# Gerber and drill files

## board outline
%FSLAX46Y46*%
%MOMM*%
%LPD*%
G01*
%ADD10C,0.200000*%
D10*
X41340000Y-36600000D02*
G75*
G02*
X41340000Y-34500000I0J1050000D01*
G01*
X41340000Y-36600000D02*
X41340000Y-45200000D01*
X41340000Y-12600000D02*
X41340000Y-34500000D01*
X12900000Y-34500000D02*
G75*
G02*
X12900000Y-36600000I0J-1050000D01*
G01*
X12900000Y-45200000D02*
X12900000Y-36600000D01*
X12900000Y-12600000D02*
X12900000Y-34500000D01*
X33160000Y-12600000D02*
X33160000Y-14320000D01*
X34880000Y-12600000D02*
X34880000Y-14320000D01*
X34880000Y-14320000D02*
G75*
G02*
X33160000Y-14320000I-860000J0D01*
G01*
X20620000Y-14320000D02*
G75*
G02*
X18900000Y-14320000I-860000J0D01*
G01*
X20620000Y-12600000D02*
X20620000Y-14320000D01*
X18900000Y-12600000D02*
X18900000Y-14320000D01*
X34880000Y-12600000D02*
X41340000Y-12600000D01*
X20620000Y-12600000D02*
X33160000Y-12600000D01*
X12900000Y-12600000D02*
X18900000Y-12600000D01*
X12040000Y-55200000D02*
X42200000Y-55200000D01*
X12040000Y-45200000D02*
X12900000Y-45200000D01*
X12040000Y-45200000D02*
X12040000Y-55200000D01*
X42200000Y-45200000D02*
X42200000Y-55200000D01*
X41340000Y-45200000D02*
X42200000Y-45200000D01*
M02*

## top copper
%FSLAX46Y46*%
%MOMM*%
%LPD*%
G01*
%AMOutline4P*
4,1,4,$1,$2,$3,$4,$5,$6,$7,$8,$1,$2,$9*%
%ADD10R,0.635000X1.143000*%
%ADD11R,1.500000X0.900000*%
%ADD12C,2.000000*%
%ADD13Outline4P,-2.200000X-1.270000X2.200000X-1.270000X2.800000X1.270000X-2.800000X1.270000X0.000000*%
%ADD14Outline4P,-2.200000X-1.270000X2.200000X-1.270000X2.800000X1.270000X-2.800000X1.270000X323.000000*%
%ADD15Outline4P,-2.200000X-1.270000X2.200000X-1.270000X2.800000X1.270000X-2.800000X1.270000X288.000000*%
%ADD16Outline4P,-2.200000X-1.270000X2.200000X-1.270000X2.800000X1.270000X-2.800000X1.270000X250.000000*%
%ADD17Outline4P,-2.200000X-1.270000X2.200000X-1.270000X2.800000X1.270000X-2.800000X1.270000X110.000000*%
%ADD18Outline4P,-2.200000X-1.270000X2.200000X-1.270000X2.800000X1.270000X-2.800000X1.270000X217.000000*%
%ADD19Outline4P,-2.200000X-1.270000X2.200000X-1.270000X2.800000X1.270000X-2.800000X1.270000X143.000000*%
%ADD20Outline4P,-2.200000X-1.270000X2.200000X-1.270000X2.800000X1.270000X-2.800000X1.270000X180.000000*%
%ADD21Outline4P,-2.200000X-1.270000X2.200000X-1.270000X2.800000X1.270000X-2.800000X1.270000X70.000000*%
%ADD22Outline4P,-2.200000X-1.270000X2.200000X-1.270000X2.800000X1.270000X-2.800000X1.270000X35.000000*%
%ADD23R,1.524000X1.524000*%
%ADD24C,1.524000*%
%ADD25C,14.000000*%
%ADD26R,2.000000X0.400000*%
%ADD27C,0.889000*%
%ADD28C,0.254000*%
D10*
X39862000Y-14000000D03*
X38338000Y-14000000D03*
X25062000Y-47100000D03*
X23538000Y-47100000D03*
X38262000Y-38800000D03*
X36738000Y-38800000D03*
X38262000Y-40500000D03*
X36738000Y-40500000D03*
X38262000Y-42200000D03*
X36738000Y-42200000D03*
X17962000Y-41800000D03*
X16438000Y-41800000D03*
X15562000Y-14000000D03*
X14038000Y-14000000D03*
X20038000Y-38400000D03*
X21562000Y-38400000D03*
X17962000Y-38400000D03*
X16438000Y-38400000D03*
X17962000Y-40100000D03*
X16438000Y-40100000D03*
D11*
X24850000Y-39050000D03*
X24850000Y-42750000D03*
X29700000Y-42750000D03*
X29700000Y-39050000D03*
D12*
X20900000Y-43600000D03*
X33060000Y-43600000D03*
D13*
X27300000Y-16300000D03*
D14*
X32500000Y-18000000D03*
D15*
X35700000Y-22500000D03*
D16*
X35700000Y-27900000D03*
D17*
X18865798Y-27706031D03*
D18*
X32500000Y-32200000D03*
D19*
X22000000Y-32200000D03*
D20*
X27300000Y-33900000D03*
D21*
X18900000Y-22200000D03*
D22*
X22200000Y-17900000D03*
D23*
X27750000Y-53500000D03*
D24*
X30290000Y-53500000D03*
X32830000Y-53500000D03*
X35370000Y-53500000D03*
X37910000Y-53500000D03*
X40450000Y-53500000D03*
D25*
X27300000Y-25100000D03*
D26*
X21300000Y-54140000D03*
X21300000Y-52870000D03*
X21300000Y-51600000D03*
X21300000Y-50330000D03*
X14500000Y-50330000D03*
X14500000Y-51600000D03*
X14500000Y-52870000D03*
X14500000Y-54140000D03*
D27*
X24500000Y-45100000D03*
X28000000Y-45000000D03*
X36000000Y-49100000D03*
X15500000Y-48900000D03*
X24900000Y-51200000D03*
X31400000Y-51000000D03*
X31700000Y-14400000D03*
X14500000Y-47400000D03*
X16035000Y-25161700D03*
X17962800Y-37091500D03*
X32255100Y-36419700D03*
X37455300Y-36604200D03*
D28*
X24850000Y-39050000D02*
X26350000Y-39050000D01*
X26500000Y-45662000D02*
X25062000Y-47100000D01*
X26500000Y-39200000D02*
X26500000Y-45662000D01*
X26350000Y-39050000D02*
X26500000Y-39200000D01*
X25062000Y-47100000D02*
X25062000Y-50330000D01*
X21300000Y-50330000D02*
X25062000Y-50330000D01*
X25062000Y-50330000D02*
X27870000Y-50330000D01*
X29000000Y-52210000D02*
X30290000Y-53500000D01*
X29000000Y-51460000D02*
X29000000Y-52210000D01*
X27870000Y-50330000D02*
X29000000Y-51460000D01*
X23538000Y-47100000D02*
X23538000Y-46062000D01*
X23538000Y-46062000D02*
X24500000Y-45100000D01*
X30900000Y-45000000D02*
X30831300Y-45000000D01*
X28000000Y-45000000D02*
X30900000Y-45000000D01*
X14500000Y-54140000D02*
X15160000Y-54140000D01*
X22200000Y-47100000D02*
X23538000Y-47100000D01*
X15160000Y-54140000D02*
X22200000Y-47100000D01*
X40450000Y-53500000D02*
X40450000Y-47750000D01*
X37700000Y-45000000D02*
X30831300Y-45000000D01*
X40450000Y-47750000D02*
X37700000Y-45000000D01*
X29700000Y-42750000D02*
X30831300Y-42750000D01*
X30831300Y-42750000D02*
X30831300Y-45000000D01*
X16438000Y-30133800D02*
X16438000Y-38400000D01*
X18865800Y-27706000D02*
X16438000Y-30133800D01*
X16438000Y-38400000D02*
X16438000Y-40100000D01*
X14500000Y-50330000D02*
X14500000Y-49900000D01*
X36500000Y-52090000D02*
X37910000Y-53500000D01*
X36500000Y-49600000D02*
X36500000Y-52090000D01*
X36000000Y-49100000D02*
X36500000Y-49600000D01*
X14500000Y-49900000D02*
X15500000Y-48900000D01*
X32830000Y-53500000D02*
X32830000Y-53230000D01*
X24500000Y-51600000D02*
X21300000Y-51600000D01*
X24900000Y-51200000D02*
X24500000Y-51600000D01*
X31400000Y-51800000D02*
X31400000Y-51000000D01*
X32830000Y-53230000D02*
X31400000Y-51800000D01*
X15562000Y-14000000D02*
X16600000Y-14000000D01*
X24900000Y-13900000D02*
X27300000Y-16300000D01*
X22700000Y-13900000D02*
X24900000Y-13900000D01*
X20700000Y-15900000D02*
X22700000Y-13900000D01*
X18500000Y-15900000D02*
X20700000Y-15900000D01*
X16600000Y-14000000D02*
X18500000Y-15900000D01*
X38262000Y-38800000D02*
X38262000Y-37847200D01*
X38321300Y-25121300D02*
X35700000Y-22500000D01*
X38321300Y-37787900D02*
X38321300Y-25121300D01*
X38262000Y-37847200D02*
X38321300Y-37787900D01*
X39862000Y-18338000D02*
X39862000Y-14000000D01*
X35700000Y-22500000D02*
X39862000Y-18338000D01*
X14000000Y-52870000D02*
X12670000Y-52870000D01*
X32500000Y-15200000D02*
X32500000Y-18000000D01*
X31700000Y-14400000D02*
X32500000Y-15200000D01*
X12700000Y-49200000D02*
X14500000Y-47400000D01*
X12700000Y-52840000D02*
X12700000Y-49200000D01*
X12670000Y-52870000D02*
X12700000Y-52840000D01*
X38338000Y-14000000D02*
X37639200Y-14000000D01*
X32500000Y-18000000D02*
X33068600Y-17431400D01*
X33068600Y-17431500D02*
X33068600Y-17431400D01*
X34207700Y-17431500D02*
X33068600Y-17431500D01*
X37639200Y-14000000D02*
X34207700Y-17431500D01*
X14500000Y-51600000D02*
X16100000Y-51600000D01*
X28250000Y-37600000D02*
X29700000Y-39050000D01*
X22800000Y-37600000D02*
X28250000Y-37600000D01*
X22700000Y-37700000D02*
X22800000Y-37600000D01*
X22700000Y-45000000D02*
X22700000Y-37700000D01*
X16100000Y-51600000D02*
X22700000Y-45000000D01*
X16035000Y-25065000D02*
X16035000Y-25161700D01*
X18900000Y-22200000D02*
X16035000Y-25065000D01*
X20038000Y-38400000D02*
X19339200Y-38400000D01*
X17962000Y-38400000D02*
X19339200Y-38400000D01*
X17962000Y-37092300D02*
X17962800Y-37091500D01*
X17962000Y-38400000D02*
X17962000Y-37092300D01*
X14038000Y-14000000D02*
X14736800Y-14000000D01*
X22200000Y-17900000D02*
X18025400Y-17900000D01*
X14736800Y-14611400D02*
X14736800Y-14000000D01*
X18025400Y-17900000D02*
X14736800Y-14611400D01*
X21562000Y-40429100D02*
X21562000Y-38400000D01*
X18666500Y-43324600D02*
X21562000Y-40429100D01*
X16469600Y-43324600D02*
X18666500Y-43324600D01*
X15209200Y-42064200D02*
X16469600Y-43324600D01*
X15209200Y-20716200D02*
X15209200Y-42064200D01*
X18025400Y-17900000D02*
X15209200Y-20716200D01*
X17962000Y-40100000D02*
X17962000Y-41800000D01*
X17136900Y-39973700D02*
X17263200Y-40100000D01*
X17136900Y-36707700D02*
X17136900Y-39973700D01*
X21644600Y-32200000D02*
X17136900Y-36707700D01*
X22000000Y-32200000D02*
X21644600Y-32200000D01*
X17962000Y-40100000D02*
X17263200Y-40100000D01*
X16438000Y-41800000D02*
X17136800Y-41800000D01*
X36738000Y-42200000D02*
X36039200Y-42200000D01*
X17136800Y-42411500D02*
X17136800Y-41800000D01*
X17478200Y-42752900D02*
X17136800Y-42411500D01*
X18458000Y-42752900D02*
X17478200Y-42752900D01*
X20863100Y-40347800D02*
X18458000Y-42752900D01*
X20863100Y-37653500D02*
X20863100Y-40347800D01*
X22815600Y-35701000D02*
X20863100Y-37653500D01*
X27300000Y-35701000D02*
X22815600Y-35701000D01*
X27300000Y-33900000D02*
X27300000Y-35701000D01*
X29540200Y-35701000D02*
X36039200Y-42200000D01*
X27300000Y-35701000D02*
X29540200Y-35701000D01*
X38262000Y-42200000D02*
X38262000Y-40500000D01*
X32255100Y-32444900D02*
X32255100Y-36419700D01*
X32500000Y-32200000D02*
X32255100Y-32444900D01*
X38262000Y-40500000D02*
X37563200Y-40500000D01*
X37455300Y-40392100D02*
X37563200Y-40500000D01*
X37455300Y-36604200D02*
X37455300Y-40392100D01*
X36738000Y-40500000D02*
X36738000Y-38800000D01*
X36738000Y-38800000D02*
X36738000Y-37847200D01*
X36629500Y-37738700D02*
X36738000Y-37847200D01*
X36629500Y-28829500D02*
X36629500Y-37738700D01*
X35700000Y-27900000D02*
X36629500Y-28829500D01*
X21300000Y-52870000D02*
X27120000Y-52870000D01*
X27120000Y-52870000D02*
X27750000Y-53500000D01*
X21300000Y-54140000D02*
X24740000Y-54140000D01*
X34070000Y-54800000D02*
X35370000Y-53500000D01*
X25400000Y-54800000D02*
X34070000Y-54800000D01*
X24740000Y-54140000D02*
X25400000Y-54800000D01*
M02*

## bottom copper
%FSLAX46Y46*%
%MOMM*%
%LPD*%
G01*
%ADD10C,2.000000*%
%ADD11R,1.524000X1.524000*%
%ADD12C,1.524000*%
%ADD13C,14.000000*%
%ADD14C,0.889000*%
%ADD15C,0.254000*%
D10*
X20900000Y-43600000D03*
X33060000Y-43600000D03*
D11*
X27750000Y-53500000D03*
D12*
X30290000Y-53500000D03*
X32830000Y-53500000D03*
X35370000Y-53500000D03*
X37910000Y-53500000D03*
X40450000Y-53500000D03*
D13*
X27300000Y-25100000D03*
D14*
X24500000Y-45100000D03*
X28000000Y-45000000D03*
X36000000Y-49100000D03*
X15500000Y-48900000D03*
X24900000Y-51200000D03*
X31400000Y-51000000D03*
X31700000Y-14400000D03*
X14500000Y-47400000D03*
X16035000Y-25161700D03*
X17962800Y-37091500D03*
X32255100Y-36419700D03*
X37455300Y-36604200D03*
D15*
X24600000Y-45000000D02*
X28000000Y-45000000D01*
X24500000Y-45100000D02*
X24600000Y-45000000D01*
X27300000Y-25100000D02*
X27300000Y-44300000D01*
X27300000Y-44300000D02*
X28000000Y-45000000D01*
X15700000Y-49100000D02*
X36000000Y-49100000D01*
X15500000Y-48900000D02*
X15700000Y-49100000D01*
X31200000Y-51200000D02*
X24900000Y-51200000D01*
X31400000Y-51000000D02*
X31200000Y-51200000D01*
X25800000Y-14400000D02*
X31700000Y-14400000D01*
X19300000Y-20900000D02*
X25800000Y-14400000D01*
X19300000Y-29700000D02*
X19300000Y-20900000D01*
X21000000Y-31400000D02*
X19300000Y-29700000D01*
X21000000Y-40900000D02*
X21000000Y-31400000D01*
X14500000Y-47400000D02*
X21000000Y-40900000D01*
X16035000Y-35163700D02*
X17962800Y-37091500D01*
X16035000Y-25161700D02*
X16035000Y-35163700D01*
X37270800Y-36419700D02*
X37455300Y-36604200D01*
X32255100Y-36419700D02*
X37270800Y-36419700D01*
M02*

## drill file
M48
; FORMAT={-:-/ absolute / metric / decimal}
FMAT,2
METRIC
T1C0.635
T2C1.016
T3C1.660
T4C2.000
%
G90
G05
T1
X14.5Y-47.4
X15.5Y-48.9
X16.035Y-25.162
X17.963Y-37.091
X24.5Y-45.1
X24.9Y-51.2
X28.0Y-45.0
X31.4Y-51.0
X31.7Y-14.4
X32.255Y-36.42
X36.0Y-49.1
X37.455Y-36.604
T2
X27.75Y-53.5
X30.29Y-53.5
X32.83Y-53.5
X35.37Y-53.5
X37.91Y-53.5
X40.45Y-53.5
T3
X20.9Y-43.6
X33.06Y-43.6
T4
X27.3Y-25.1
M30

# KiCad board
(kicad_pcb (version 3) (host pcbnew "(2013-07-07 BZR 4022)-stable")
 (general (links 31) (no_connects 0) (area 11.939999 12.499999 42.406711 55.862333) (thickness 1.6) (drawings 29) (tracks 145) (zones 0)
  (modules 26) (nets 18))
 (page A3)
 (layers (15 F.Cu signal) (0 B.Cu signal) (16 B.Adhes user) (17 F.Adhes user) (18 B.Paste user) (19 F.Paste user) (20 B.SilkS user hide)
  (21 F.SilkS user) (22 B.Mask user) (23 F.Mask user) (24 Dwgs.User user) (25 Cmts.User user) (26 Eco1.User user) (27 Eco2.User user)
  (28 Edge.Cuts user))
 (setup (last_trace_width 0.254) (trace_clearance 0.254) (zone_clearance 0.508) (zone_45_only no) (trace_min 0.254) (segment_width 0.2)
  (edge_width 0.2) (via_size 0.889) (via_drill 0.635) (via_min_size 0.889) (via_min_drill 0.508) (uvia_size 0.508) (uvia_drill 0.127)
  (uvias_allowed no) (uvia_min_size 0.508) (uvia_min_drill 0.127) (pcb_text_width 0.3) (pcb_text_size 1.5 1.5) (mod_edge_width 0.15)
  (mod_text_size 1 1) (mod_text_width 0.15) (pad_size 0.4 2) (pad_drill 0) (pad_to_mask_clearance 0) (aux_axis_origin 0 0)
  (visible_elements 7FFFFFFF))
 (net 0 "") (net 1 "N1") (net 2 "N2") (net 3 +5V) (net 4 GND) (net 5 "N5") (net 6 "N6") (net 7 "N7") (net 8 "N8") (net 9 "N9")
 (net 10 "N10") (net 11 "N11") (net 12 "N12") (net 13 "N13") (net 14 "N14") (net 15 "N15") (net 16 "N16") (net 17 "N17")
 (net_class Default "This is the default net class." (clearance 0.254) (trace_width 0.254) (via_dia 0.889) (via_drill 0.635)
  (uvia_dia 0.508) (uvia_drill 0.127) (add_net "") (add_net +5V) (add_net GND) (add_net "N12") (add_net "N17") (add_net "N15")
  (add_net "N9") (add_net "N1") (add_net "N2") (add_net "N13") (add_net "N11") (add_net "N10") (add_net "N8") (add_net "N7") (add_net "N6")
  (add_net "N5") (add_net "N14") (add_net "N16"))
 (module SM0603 (layer F.Cu) (at 39.1 14 180)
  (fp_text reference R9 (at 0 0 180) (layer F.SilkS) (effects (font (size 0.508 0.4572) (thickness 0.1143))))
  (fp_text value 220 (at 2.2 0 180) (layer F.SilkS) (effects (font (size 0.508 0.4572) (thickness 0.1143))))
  (pad 1 smd rect (at -0.762 0 180) (size 0.635 1.143) (layers F.Cu F.Paste F.Mask) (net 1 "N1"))
  (pad 2 smd rect (at 0.762 0 180) (size 0.635 1.143) (layers F.Cu F.Paste F.Mask) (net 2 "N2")))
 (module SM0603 (layer F.Cu) (at 24.3 47.1 180)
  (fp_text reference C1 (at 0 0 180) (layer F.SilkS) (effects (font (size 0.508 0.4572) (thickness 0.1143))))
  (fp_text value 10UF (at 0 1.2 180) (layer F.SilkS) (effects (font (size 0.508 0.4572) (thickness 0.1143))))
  (pad 1 smd rect (at -0.762 0 180) (size 0.635 1.143) (layers F.Cu F.Paste F.Mask) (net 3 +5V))
  (pad 2 smd rect (at 0.762 0 180) (size 0.635 1.143) (layers F.Cu F.Paste F.Mask) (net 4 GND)))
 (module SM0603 (layer F.Cu) (at 37.5 38.8 180)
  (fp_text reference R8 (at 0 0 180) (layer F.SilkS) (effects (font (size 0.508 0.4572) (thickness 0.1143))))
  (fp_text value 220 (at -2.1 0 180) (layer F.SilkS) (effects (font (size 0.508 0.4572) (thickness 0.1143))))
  (pad 1 smd rect (at -0.762 0 180) (size 0.635 1.143) (layers F.Cu F.Paste F.Mask) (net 1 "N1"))
  (pad 2 smd rect (at 0.762 0 180) (size 0.635 1.143) (layers F.Cu F.Paste F.Mask) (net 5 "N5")))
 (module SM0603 (layer F.Cu) (at 37.5 40.5 180)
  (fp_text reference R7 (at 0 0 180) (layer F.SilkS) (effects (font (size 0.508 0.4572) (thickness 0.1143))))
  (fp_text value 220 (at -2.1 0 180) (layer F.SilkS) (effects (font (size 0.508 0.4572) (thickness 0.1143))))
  (pad 1 smd rect (at -0.762 0 180) (size 0.635 1.143) (layers F.Cu F.Paste F.Mask) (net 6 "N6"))
  (pad 2 smd rect (at 0.762 0 180) (size 0.635 1.143) (layers F.Cu F.Paste F.Mask) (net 5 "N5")))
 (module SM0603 (layer F.Cu) (at 37.5 42.2 180)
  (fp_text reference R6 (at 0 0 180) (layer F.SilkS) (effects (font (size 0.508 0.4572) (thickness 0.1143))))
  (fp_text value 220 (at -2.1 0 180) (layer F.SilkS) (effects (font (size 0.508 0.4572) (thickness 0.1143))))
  (pad 1 smd rect (at -0.762 0 180) (size 0.635 1.143) (layers F.Cu F.Paste F.Mask) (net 6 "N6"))
  (pad 2 smd rect (at 0.762 0 180) (size 0.635 1.143) (layers F.Cu F.Paste F.Mask) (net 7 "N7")))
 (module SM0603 (layer F.Cu) (at 17.2 41.8 180)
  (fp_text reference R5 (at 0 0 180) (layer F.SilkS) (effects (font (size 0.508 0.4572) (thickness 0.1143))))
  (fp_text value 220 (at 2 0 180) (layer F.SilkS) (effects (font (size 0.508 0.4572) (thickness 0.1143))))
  (pad 1 smd rect (at -0.762 0 180) (size 0.635 1.143) (layers F.Cu F.Paste F.Mask) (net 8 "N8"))
  (pad 2 smd rect (at 0.762 0 180) (size 0.635 1.143) (layers F.Cu F.Paste F.Mask) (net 7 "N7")))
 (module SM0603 (layer F.Cu) (at 14.8 14 180)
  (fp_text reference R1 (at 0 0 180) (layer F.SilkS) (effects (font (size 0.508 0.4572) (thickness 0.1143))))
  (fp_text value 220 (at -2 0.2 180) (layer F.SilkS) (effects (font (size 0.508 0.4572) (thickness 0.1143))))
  (pad 1 smd rect (at -0.762 0 180) (size 0.635 1.143) (layers F.Cu F.Paste F.Mask) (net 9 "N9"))
  (pad 2 smd rect (at 0.762 0 180) (size 0.635 1.143) (layers F.Cu F.Paste F.Mask) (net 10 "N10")))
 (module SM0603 (layer F.Cu) (at 20.8 38.4)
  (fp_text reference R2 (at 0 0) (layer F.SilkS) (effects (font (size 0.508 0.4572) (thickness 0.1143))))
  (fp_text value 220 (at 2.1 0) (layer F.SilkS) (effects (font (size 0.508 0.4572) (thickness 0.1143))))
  (pad 1 smd rect (at -0.762 0) (size 0.635 1.143) (layers F.Cu F.Paste F.Mask) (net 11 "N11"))
  (pad 2 smd rect (at 0.762 0) (size 0.635 1.143) (layers F.Cu F.Paste F.Mask) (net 10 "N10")))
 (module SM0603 (layer F.Cu) (at 17.2 38.4 180)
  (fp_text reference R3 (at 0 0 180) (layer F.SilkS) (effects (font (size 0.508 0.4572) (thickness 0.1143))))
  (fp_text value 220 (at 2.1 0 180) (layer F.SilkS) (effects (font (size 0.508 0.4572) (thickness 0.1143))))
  (pad 1 smd rect (at -0.762 0 180) (size 0.635 1.143) (layers F.Cu F.Paste F.Mask) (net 11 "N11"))
  (pad 2 smd rect (at 0.762 0 180) (size 0.635 1.143) (layers F.Cu F.Paste F.Mask) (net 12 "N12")))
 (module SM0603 (layer F.Cu) (at 17.2 40.1 180)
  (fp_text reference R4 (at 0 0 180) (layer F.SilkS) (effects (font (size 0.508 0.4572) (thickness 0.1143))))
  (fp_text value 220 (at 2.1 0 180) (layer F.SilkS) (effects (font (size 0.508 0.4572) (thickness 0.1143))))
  (pad 1 smd rect (at -0.762 0 180) (size 0.635 1.143) (layers F.Cu F.Paste F.Mask) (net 8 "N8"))
  (pad 2 smd rect (at 0.762 0 180) (size 0.635 1.143) (layers F.Cu F.Paste F.Mask) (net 12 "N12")))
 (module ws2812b (layer F.Cu) (at 27.3 40.9)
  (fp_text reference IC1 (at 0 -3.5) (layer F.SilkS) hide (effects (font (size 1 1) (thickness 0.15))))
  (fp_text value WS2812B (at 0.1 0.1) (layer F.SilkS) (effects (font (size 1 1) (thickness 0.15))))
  (pad 1 smd rect (at -2.45 -1.85) (size 1.5 0.9) (layers F.Cu F.Paste F.Mask) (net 3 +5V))
  (pad 2 smd rect (at -2.45 1.85) (size 1.5 0.9) (layers F.Cu F.Paste F.Mask))
  (pad 3 smd rect (at 2.4 1.85) (size 1.5 0.9) (layers F.Cu F.Paste F.Mask) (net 4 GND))
  (pad 4 smd rect (at 2.4 -1.85) (size 1.5 0.9) (layers F.Cu F.Paste F.Mask) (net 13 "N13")))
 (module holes (layer F.Cu) (at 20.9 43.6)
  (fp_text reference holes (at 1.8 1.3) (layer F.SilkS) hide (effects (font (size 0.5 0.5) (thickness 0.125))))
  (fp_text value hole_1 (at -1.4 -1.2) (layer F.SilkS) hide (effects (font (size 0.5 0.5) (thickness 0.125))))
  (pad 2 thru_hole circle (at 0 0) (size 2 2) (drill 1.66) (layers *.Cu *.Mask F.SilkS)))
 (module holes (layer F.Cu) (at 33.1 43.6)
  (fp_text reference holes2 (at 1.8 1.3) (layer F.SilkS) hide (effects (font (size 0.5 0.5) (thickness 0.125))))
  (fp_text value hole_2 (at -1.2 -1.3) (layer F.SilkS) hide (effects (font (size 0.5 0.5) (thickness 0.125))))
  (pad 2 thru_hole circle (at -0.04 0) (size 2 2) (drill 1.66) (layers *.Cu *.Mask F.SilkS)))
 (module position (layer F.Cu) (at 27.4 16.3)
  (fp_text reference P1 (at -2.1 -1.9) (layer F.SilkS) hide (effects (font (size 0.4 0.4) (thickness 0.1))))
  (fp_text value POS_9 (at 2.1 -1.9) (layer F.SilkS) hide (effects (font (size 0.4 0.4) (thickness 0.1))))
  (pad 1 smd trapezoid (at -0.1 0) (size 5 2.54) (rect_delta 0 -0.6) (layers F.Cu F.Paste F.Mask) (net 9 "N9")))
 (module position (layer F.Cu) (at 32.5 18 323)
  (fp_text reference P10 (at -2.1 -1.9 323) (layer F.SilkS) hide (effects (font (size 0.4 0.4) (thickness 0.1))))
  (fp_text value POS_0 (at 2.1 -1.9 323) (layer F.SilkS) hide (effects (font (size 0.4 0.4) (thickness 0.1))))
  (pad 1 smd trapezoid (at 0 0 323) (size 5 2.54) (rect_delta 0 -0.6) (layers F.Cu F.Paste F.Mask) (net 2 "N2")))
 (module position (layer F.Cu) (at 35.7 22.5 288)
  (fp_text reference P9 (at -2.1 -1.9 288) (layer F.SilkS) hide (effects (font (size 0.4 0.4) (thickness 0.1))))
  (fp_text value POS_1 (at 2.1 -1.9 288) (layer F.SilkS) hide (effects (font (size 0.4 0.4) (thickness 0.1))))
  (pad 1 smd trapezoid (at 0 0 288) (size 5 2.54) (rect_delta 0 -0.6) (layers F.Cu F.Paste F.Mask) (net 1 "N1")))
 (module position (layer F.Cu) (at 35.7 27.9 250)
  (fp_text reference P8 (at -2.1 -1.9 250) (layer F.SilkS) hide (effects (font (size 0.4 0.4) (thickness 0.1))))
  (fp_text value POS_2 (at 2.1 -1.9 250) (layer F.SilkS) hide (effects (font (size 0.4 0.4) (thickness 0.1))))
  (pad 1 smd trapezoid (at 0 0 250) (size 5 2.54) (rect_delta 0 -0.6) (layers F.Cu F.Paste F.Mask) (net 5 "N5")))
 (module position (layer F.Cu) (at 18.9 27.8 110)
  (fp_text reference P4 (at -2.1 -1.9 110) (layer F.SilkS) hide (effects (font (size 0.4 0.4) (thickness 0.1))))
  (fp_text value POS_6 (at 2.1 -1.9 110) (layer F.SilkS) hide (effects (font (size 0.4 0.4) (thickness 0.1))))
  (pad 1 smd trapezoid (at 0.1 0 110) (size 5 2.54) (rect_delta 0 -0.6) (layers F.Cu F.Paste F.Mask) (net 12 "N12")))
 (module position (layer F.Cu) (at 32.5 32.2 217)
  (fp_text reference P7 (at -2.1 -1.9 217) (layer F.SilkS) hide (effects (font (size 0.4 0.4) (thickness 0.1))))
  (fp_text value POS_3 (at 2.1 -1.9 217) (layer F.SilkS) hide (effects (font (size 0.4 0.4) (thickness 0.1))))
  (pad 1 smd trapezoid (at 0 0 217) (size 5 2.54) (rect_delta 0 -0.6) (layers F.Cu F.Paste F.Mask) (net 6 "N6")))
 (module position (layer F.Cu) (at 22 32.2 143)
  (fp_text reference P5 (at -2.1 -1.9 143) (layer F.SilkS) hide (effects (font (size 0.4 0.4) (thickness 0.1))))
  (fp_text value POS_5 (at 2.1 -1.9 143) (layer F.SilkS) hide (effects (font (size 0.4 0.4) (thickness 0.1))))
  (pad 1 smd trapezoid (at 0 0 143) (size 5 2.54) (rect_delta 0 -0.6) (layers F.Cu F.Paste F.Mask) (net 8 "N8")))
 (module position (layer F.Cu) (at 27.3 33.9 180)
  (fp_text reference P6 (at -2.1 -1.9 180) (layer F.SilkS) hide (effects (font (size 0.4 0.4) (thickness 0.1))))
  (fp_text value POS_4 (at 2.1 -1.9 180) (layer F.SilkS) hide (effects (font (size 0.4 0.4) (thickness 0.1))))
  (pad 1 smd trapezoid (at 0 0 180) (size 5 2.54) (rect_delta 0 -0.6) (layers F.Cu F.Paste F.Mask) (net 7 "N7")))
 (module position (layer F.Cu) (at 18.9 22.2 70)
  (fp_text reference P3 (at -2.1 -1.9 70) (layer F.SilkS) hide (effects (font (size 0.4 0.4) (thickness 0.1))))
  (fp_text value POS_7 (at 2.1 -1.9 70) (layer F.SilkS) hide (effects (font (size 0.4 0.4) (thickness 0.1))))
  (pad 1 smd trapezoid (at 0 0 70) (size 5 2.54) (rect_delta 0 -0.6) (layers F.Cu F.Paste F.Mask) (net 11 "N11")))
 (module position (layer F.Cu) (at 22.2 17.9 35)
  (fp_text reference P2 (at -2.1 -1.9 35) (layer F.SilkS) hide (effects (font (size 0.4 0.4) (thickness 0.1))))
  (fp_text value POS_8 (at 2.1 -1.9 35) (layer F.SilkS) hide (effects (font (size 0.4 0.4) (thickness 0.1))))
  (pad 1 smd trapezoid (at 0 0 35) (size 5 2.54) (rect_delta 0 -0.6) (layers F.Cu F.Paste F.Mask) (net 10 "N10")))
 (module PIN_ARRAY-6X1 (layer F.Cu) (at 34.1 53.5)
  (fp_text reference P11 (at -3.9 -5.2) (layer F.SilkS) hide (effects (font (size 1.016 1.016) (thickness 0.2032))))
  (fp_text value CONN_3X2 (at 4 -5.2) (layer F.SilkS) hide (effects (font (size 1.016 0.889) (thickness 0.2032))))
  (pad 1 thru_hole rect (at -6.35 0) (size 1.524 1.524) (drill 1.016) (layers *.Cu *.Mask F.SilkS) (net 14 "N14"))
  (pad 2 thru_hole circle (at -3.81 0) (size 1.524 1.524) (drill 1.016) (layers *.Cu *.Mask F.SilkS) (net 3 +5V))
  (pad 3 thru_hole circle (at -1.27 0) (size 1.524 1.524) (drill 1.016) (layers *.Cu *.Mask F.SilkS) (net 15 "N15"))
  (pad 4 thru_hole circle (at 1.27 0) (size 1.524 1.524) (drill 1.016) (layers *.Cu *.Mask F.SilkS) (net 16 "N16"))
  (pad 5 thru_hole circle (at 3.81 0) (size 1.524 1.524) (drill 1.016) (layers *.Cu *.Mask F.SilkS) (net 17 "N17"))
  (pad 6 thru_hole circle (at 6.35 0) (size 1.524 1.524) (drill 1.016) (layers *.Cu *.Mask F.SilkS) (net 4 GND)))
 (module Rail (layer F.Cu) (at 27.3 25.1 90)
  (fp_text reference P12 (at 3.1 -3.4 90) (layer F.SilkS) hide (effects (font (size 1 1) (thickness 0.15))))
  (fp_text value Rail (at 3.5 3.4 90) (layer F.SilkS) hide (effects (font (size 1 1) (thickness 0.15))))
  (pad 1 thru_hole circle (at 0 0 90) (size 14 14) (drill 2) (layers *.Cu *.Mask F.SilkS) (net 4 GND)))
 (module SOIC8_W (layer F.Cu) (at 18 52.2 270)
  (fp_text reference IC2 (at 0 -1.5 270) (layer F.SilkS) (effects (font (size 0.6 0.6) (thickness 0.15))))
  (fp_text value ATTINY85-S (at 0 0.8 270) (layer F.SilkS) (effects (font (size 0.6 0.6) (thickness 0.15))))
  (pad 5 smd rect (at 1.94 -3.3 270) (size 0.4 2) (layers F.Cu F.Paste F.Mask) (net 16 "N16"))
  (pad 6 smd rect (at 0.67 -3.3 270) (size 0.4 2) (layers F.Cu F.Paste F.Mask) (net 14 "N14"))
  (pad 7 smd rect (at -0.6 -3.3 270) (size 0.4 2) (layers F.Cu F.Paste F.Mask) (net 15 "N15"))
  (pad 8 smd rect (at -1.87 -3.3 270) (size 0.4 2) (layers F.Cu F.Paste F.Mask) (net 3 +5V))
  (pad 1 smd rect (at -1.87 3.5 270) (size 0.4 2) (layers F.Cu F.Paste F.Mask) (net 17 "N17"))
  (pad 2 smd rect (at -0.6 3.5 270) (size 0.4 2) (layers F.Cu F.Paste F.Mask) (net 13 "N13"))
  (pad 3 smd rect (at 0.67 3.5 270) (size 0.4 2) (layers F.Cu F.Paste F.Mask) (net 2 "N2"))
  (pad 4 smd rect (at 1.94 3.5 270) (size 0.4 2) (layers F.Cu F.Paste F.Mask) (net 4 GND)))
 (gr_arc (start 41.34 35.55) (end 41.34 34.5) (angle -180) (layer Edge.Cuts) (width 0.2))
 (gr_line (start 41.34 36.6) (end 41.34 45.2) (angle 90) (layer Edge.Cuts) (width 0.2))
 (gr_line (start 41.34 12.6) (end 41.34 34.5) (angle 90) (layer Edge.Cuts) (width 0.2))
 (gr_arc (start 12.9 35.55) (end 12.9 34.5) (angle 180) (layer Edge.Cuts) (width 0.2))
 (gr_line (start 12.9 45.2) (end 12.9 36.6) (angle 90) (layer Edge.Cuts) (width 0.2))
 (gr_line (start 12.9 12.6) (end 12.9 34.5) (angle 90) (layer Edge.Cuts) (width 0.2))
 (gr_line (start 33.16 12.6) (end 33.16 14.32) (angle 90) (layer Edge.Cuts) (width 0.2))
 (gr_line (start 34.88 12.6) (end 34.88 14.32) (angle 90) (layer Edge.Cuts) (width 0.2))
 (gr_arc (start 34.02 14.32) (end 33.16 14.32) (angle -180) (layer Edge.Cuts) (width 0.2))
 (gr_arc (start 19.76 14.32) (end 18.9 14.32) (angle -180) (layer Edge.Cuts) (width 0.2))
 (gr_line (start 20.62 12.6) (end 20.62 14.32) (angle 90) (layer Edge.Cuts) (width 0.2))
 (gr_line (start 18.9 12.6) (end 18.9 14.32) (angle 90) (layer Edge.Cuts) (width 0.2))
 (gr_line (start 34.88 12.6) (end 41.34 12.6) (angle 90) (layer Edge.Cuts) (width 0.2))
 (gr_line (start 20.62 12.6) (end 33.16 12.6) (angle 90) (layer Edge.Cuts) (width 0.2))
 (gr_line (start 12.9 12.6) (end 18.9 12.6) (angle 90) (layer Edge.Cuts) (width 0.2))
 (gr_line (start 12.04 55.2) (end 42.2 55.2) (angle 90) (layer Edge.Cuts) (width 0.2))
 (gr_line (start 12.04 45.2) (end 12.9 45.2) (angle 90) (layer Edge.Cuts) (width 0.2))
 (gr_line (start 12.04 45.2) (end 12.04 55.2) (angle 90) (layer Edge.Cuts) (width 0.2))
 (gr_line (start 42.2 45.2) (end 42.2 55.2) (angle 90) (layer Edge.Cuts) (width 0.2))
 (gr_line (start 41.34 45.2) (end 42.2 45.2) (angle 90) (layer Edge.Cuts) (width 0.2))
 (segment (start 24.85 39.05) (end 26.35 39.05) (width 0.254) (layer F.Cu) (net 3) (status 400000))
 (segment (start 26.5 45.662) (end 25.062 47.1) (width 0.254) (layer F.Cu) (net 3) (status 800000))
 (segment (start 26.5 39.2) (end 26.5 45.662) (width 0.254) (layer F.Cu) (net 3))
 (segment (start 26.35 39.05) (end 26.5 39.2) (width 0.254) (layer F.Cu) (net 3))
 (segment (start 25.062 47.1) (end 25.062 50.33) (width 0.254) (layer F.Cu) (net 3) (status 400000))
 (segment (start 21.3 50.33) (end 25.062 50.33) (width 0.254) (layer F.Cu) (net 3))
 (segment (start 25.062 50.33) (end 27.87 50.33) (width 0.254) (layer F.Cu) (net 3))
 (segment (start 29 52.21) (end 30.29 53.5) (width 0.254) (layer F.Cu) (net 3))
 (segment (start 29 51.46) (end 29 52.21) (width 0.254) (layer F.Cu) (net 3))
 (segment (start 27.87 50.33) (end 29 51.46) (width 0.254) (layer F.Cu) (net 3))
 (segment (start 23.538 47.1) (end 23.538 46.062) (width 0.254) (layer F.Cu) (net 4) (status 400000))
 (segment (start 24.6 45) (end 28 45) (width 0.254) (layer B.Cu) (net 4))
 (segment (start 24.5 45.1) (end 24.6 45) (width 0.254) (layer B.Cu) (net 4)) (via (at 24.5 45.1) (size 0.889) (layers F.Cu B.Cu) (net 4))
 (segment (start 23.538 46.062) (end 24.5 45.1) (width 0.254) (layer F.Cu) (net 4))
 (segment (start 27.3 25.1) (end 27.3 44.3) (width 0.254) (layer B.Cu) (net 4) (status 400000))
 (segment (start 27.3 44.3) (end 28 45) (width 0.254) (layer B.Cu) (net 4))
 (segment (start 30.9 45) (end 30.8313 45) (width 0.254) (layer F.Cu) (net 4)) (via (at 28 45) (size 0.889) (layers F.Cu B.Cu) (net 4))
 (segment (start 28 45) (end 30.9 45) (width 0.254) (layer F.Cu) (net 4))
 (segment (start 14.5 54.14) (end 15.16 54.14) (width 0.254) (layer F.Cu) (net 4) (status C00000))
 (segment (start 22.2 47.1) (end 23.538 47.1) (width 0.254) (layer F.Cu) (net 4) (status 800000))
 (segment (start 15.16 54.14) (end 22.2 47.1) (width 0.254) (layer F.Cu) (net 4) (status 400000))
 (segment (start 40.45 53.5) (end 40.45 47.75) (width 0.254) (layer F.Cu) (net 4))
 (segment (start 37.7 45) (end 30.8313 45) (width 0.254) (layer F.Cu) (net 4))
 (segment (start 40.45 47.75) (end 37.7 45) (width 0.254) (layer F.Cu) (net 4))
 (segment (start 29.7 42.75) (end 30.8313 42.75) (width 0.254) (layer F.Cu) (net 4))
 (segment (start 30.8313 42.75) (end 30.8313 45) (width 0.254) (layer F.Cu) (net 4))
 (segment (start 16.438 30.1338) (end 16.438 38.4) (width 0.254) (layer F.Cu) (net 12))
 (segment (start 18.8658 27.706) (end 16.438 30.1338) (width 0.254) (layer F.Cu) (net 12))
 (segment (start 16.438 38.4) (end 16.438 40.1) (width 0.254) (layer F.Cu) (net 12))
 (segment (start 14.5 50.33) (end 14.5 49.9) (width 0.254) (layer F.Cu) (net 17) (status 400000))
 (segment (start 36.5 52.09) (end 37.91 53.5) (width 0.254) (layer F.Cu) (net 17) (status 800000))
 (segment (start 36.5 49.6) (end 36.5 52.09) (width 0.254) (layer F.Cu) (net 17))
 (segment (start 36 49.1) (end 36.5 49.6) (width 0.254) (layer F.Cu) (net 17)) (via (at 36 49.1) (size 0.889) (layers F.Cu B.Cu) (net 17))
 (segment (start 15.7 49.1) (end 36 49.1) (width 0.254) (layer B.Cu) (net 17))
 (segment (start 15.5 48.9) (end 15.7 49.1) (width 0.254) (layer B.Cu) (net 17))
 (via (at 15.5 48.9) (size 0.889) (layers F.Cu B.Cu) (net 17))
 (segment (start 14.5 49.9) (end 15.5 48.9) (width 0.254) (layer F.Cu) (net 17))
 (segment (start 32.83 53.5) (end 32.83 53.23) (width 0.254) (layer F.Cu) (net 15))
 (segment (start 24.5 51.6) (end 21.3 51.6) (width 0.254) (layer F.Cu) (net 15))
 (segment (start 24.9 51.2) (end 24.5 51.6) (width 0.254) (layer F.Cu) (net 15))
 (via (at 24.9 51.2) (size 0.889) (layers F.Cu B.Cu) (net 15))
 (segment (start 31.2 51.2) (end 24.9 51.2) (width 0.254) (layer B.Cu) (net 15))
 (segment (start 31.4 51) (end 31.2 51.2) (width 0.254) (layer B.Cu) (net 15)) (via (at 31.4 51) (size 0.889) (layers F.Cu B.Cu) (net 15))
 (segment (start 31.4 51.8) (end 31.4 51) (width 0.254) (layer F.Cu) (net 15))
 (segment (start 32.83 53.23) (end 31.4 51.8) (width 0.254) (layer F.Cu) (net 15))
 (segment (start 15.562 14) (end 16.6 14) (width 0.254) (layer F.Cu) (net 9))
 (segment (start 24.9 13.9) (end 27.3 16.3) (width 0.254) (layer F.Cu) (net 9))
 (segment (start 22.7 13.9) (end 24.9 13.9) (width 0.254) (layer F.Cu) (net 9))
 (segment (start 20.7 15.9) (end 22.7 13.9) (width 0.254) (layer F.Cu) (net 9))
 (segment (start 18.5 15.9) (end 20.7 15.9) (width 0.254) (layer F.Cu) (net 9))
 (segment (start 16.6 14) (end 18.5 15.9) (width 0.254) (layer F.Cu) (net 9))
 (segment (start 38.262 38.8) (end 38.262 37.8472) (width 0.254) (layer F.Cu) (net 1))
 (segment (start 38.3213 25.1213) (end 35.7 22.5) (width 0.254) (layer F.Cu) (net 1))
 (segment (start 38.3213 37.7879) (end 38.3213 25.1213) (width 0.254) (layer F.Cu) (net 1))
 (segment (start 38.262 37.8472) (end 38.3213 37.7879) (width 0.254) (layer F.Cu) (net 1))
 (segment (start 39.862 18.338) (end 39.862 14) (width 0.254) (layer F.Cu) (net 1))
 (segment (start 35.7 22.5) (end 39.862 18.338) (width 0.254) (layer F.Cu) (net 1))
 (segment (start 14 52.87) (end 12.67 52.87) (width 0.254) (layer F.Cu) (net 2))
 (segment (start 32.5 15.2) (end 32.5 18) (width 0.254) (layer F.Cu) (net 2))
 (segment (start 31.7 14.4) (end 32.5 15.2) (width 0.254) (layer F.Cu) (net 2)) (via (at 31.7 14.4) (size 0.889) (layers F.Cu B.Cu) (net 2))
 (segment (start 25.8 14.4) (end 31.7 14.4) (width 0.254) (layer B.Cu) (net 2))
 (segment (start 19.3 20.9) (end 25.8 14.4) (width 0.254) (layer B.Cu) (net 2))
 (segment (start 19.3 29.7) (end 19.3 20.9) (width 0.254) (layer B.Cu) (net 2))
 (segment (start 21 31.4) (end 19.3 29.7) (width 0.254) (layer B.Cu) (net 2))
 (segment (start 21 40.9) (end 21 31.4) (width 0.254) (layer B.Cu) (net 2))
 (segment (start 14.5 47.4) (end 21 40.9) (width 0.254) (layer B.Cu) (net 2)) (via (at 14.5 47.4) (size 0.889) (layers F.Cu B.Cu) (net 2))
 (segment (start 12.7 49.2) (end 14.5 47.4) (width 0.254) (layer F.Cu) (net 2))
 (segment (start 12.7 52.84) (end 12.7 49.2) (width 0.254) (layer F.Cu) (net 2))
 (segment (start 12.67 52.87) (end 12.7 52.84) (width 0.254) (layer F.Cu) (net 2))
 (segment (start 38.338 14) (end 37.6392 14) (width 0.254) (layer F.Cu) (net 2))
 (segment (start 32.5 18) (end 33.0686 17.4314) (width 0.254) (layer F.Cu) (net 2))
 (segment (start 33.0686 17.4315) (end 33.0686 17.4314) (width 0.254) (layer F.Cu) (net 2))
 (segment (start 34.2077 17.4315) (end 33.0686 17.4315) (width 0.254) (layer F.Cu) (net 2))
 (segment (start 37.6392 14) (end 34.2077 17.4315) (width 0.254) (layer F.Cu) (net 2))
 (segment (start 14.5 51.6) (end 16.1 51.6) (width 0.254) (layer F.Cu) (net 13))
 (segment (start 28.25 37.6) (end 29.7 39.05) (width 0.254) (layer F.Cu) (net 13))
 (segment (start 22.8 37.6) (end 28.25 37.6) (width 0.254) (layer F.Cu) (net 13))
 (segment (start 22.7 37.7) (end 22.8 37.6) (width 0.254) (layer F.Cu) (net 13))
 (segment (start 22.7 45) (end 22.7 37.7) (width 0.254) (layer F.Cu) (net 13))
 (segment (start 16.1 51.6) (end 22.7 45) (width 0.254) (layer F.Cu) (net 13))
 (via (at 16.035 25.1617) (size 0.889) (layers F.Cu B.Cu) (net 11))
 (via (at 17.9628 37.0915) (size 0.889) (layers F.Cu B.Cu) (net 11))
 (segment (start 16.035 25.065) (end 16.035 25.1617) (width 0.254) (layer F.Cu) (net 11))
 (segment (start 18.9 22.2) (end 16.035 25.065) (width 0.254) (layer F.Cu) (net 11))
 (segment (start 20.038 38.4) (end 19.3392 38.4) (width 0.254) (layer F.Cu) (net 11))
 (segment (start 17.962 38.4) (end 19.3392 38.4) (width 0.254) (layer F.Cu) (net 11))
 (segment (start 16.035 35.1637) (end 17.9628 37.0915) (width 0.254) (layer B.Cu) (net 11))
 (segment (start 16.035 25.1617) (end 16.035 35.1637) (width 0.254) (layer B.Cu) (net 11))
 (segment (start 17.962 37.0923) (end 17.9628 37.0915) (width 0.254) (layer F.Cu) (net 11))
 (segment (start 17.962 38.4) (end 17.962 37.0923) (width 0.254) (layer F.Cu) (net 11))
 (segment (start 14.038 14) (end 14.7368 14) (width 0.254) (layer F.Cu) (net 10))
 (segment (start 22.2 17.9) (end 18.0254 17.9) (width 0.254) (layer F.Cu) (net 10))
 (segment (start 14.7368 14.6114) (end 14.7368 14) (width 0.254) (layer F.Cu) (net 10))
 (segment (start 18.0254 17.9) (end 14.7368 14.6114) (width 0.254) (layer F.Cu) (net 10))
 (segment (start 21.562 40.4291) (end 21.562 38.4) (width 0.254) (layer F.Cu) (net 10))
 (segment (start 18.6665 43.3246) (end 21.562 40.4291) (width 0.254) (layer F.Cu) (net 10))
 (segment (start 16.4696 43.3246) (end 18.6665 43.3246) (width 0.254) (layer F.Cu) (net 10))
 (segment (start 15.2092 42.0642) (end 16.4696 43.3246) (width 0.254) (layer F.Cu) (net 10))
 (segment (start 15.2092 20.7162) (end 15.2092 42.0642) (width 0.254) (layer F.Cu) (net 10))
 (segment (start 18.0254 17.9) (end 15.2092 20.7162) (width 0.254) (layer F.Cu) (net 10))
 (segment (start 17.962 40.1) (end 17.962 41.8) (width 0.254) (layer F.Cu) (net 8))
 (segment (start 17.1369 39.9737) (end 17.2632 40.1) (width 0.254) (layer F.Cu) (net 8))
 (segment (start 17.1369 36.7077) (end 17.1369 39.9737) (width 0.254) (layer F.Cu) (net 8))
 (segment (start 21.6446 32.2) (end 17.1369 36.7077) (width 0.254) (layer F.Cu) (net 8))
 (segment (start 22 32.2) (end 21.6446 32.2) (width 0.254) (layer F.Cu) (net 8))
 (segment (start 17.962 40.1) (end 17.2632 40.1) (width 0.254) (layer F.Cu) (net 8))
 (segment (start 16.438 41.8) (end 17.1368 41.8) (width 0.254) (layer F.Cu) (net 7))
 (segment (start 36.738 42.2) (end 36.0392 42.2) (width 0.254) (layer F.Cu) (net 7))
 (segment (start 17.1368 42.4115) (end 17.1368 41.8) (width 0.254) (layer F.Cu) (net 7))
 (segment (start 17.4782 42.7529) (end 17.1368 42.4115) (width 0.254) (layer F.Cu) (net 7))
 (segment (start 18.458 42.7529) (end 17.4782 42.7529) (width 0.254) (layer F.Cu) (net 7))
 (segment (start 20.8631 40.3478) (end 18.458 42.7529) (width 0.254) (layer F.Cu) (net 7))
 (segment (start 20.8631 37.6535) (end 20.8631 40.3478) (width 0.254) (layer F.Cu) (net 7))
 (segment (start 22.8156 35.701) (end 20.8631 37.6535) (width 0.254) (layer F.Cu) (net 7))
 (segment (start 27.3 35.701) (end 22.8156 35.701) (width 0.254) (layer F.Cu) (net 7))
 (segment (start 27.3 33.9) (end 27.3 35.701) (width 0.254) (layer F.Cu) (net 7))
 (segment (start 29.5402 35.701) (end 36.0392 42.2) (width 0.254) (layer F.Cu) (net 7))
 (segment (start 27.3 35.701) (end 29.5402 35.701) (width 0.254) (layer F.Cu) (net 7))
 (via (at 32.2551 36.4197) (size 0.889) (layers F.Cu B.Cu) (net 6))
 (via (at 37.4553 36.6042) (size 0.889) (layers F.Cu B.Cu) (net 6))
 (segment (start 38.262 42.2) (end 38.262 40.5) (width 0.254) (layer F.Cu) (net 6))
 (segment (start 32.2551 32.4449) (end 32.2551 36.4197) (width 0.254) (layer F.Cu) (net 6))
 (segment (start 32.5 32.2) (end 32.2551 32.4449) (width 0.254) (layer F.Cu) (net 6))
 (segment (start 38.262 40.5) (end 37.5632 40.5) (width 0.254) (layer F.Cu) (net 6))
 (segment (start 37.2708 36.4197) (end 37.4553 36.6042) (width 0.254) (layer B.Cu) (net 6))
 (segment (start 32.2551 36.4197) (end 37.2708 36.4197) (width 0.254) (layer B.Cu) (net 6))
 (segment (start 37.4553 40.3921) (end 37.5632 40.5) (width 0.254) (layer F.Cu) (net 6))
 (segment (start 37.4553 36.6042) (end 37.4553 40.3921) (width 0.254) (layer F.Cu) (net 6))
 (segment (start 36.738 40.5) (end 36.738 38.8) (width 0.254) (layer F.Cu) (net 5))
 (segment (start 36.738 38.8) (end 36.738 37.8472) (width 0.254) (layer F.Cu) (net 5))
 (segment (start 36.6295 37.7387) (end 36.738 37.8472) (width 0.254) (layer F.Cu) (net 5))
 (segment (start 36.6295 28.8295) (end 36.6295 37.7387) (width 0.254) (layer F.Cu) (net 5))
 (segment (start 35.7 27.9) (end 36.6295 28.8295) (width 0.254) (layer F.Cu) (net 5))
 (segment (start 21.3 52.87) (end 27.12 52.87) (width 0.254) (layer F.Cu) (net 14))
 (segment (start 27.12 52.87) (end 27.75 53.5) (width 0.254) (layer F.Cu) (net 14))
 (segment (start 21.3 54.14) (end 24.74 54.14) (width 0.254) (layer F.Cu) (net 16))
 (segment (start 34.07 54.8) (end 35.37 53.5) (width 0.254) (layer F.Cu) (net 16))
 (segment (start 25.4 54.8) (end 34.07 54.8) (width 0.254) (layer F.Cu) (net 16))
 (segment (start 24.74 54.14) (end 25.4 54.8) (width 0.254) (layer F.Cu) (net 16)))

